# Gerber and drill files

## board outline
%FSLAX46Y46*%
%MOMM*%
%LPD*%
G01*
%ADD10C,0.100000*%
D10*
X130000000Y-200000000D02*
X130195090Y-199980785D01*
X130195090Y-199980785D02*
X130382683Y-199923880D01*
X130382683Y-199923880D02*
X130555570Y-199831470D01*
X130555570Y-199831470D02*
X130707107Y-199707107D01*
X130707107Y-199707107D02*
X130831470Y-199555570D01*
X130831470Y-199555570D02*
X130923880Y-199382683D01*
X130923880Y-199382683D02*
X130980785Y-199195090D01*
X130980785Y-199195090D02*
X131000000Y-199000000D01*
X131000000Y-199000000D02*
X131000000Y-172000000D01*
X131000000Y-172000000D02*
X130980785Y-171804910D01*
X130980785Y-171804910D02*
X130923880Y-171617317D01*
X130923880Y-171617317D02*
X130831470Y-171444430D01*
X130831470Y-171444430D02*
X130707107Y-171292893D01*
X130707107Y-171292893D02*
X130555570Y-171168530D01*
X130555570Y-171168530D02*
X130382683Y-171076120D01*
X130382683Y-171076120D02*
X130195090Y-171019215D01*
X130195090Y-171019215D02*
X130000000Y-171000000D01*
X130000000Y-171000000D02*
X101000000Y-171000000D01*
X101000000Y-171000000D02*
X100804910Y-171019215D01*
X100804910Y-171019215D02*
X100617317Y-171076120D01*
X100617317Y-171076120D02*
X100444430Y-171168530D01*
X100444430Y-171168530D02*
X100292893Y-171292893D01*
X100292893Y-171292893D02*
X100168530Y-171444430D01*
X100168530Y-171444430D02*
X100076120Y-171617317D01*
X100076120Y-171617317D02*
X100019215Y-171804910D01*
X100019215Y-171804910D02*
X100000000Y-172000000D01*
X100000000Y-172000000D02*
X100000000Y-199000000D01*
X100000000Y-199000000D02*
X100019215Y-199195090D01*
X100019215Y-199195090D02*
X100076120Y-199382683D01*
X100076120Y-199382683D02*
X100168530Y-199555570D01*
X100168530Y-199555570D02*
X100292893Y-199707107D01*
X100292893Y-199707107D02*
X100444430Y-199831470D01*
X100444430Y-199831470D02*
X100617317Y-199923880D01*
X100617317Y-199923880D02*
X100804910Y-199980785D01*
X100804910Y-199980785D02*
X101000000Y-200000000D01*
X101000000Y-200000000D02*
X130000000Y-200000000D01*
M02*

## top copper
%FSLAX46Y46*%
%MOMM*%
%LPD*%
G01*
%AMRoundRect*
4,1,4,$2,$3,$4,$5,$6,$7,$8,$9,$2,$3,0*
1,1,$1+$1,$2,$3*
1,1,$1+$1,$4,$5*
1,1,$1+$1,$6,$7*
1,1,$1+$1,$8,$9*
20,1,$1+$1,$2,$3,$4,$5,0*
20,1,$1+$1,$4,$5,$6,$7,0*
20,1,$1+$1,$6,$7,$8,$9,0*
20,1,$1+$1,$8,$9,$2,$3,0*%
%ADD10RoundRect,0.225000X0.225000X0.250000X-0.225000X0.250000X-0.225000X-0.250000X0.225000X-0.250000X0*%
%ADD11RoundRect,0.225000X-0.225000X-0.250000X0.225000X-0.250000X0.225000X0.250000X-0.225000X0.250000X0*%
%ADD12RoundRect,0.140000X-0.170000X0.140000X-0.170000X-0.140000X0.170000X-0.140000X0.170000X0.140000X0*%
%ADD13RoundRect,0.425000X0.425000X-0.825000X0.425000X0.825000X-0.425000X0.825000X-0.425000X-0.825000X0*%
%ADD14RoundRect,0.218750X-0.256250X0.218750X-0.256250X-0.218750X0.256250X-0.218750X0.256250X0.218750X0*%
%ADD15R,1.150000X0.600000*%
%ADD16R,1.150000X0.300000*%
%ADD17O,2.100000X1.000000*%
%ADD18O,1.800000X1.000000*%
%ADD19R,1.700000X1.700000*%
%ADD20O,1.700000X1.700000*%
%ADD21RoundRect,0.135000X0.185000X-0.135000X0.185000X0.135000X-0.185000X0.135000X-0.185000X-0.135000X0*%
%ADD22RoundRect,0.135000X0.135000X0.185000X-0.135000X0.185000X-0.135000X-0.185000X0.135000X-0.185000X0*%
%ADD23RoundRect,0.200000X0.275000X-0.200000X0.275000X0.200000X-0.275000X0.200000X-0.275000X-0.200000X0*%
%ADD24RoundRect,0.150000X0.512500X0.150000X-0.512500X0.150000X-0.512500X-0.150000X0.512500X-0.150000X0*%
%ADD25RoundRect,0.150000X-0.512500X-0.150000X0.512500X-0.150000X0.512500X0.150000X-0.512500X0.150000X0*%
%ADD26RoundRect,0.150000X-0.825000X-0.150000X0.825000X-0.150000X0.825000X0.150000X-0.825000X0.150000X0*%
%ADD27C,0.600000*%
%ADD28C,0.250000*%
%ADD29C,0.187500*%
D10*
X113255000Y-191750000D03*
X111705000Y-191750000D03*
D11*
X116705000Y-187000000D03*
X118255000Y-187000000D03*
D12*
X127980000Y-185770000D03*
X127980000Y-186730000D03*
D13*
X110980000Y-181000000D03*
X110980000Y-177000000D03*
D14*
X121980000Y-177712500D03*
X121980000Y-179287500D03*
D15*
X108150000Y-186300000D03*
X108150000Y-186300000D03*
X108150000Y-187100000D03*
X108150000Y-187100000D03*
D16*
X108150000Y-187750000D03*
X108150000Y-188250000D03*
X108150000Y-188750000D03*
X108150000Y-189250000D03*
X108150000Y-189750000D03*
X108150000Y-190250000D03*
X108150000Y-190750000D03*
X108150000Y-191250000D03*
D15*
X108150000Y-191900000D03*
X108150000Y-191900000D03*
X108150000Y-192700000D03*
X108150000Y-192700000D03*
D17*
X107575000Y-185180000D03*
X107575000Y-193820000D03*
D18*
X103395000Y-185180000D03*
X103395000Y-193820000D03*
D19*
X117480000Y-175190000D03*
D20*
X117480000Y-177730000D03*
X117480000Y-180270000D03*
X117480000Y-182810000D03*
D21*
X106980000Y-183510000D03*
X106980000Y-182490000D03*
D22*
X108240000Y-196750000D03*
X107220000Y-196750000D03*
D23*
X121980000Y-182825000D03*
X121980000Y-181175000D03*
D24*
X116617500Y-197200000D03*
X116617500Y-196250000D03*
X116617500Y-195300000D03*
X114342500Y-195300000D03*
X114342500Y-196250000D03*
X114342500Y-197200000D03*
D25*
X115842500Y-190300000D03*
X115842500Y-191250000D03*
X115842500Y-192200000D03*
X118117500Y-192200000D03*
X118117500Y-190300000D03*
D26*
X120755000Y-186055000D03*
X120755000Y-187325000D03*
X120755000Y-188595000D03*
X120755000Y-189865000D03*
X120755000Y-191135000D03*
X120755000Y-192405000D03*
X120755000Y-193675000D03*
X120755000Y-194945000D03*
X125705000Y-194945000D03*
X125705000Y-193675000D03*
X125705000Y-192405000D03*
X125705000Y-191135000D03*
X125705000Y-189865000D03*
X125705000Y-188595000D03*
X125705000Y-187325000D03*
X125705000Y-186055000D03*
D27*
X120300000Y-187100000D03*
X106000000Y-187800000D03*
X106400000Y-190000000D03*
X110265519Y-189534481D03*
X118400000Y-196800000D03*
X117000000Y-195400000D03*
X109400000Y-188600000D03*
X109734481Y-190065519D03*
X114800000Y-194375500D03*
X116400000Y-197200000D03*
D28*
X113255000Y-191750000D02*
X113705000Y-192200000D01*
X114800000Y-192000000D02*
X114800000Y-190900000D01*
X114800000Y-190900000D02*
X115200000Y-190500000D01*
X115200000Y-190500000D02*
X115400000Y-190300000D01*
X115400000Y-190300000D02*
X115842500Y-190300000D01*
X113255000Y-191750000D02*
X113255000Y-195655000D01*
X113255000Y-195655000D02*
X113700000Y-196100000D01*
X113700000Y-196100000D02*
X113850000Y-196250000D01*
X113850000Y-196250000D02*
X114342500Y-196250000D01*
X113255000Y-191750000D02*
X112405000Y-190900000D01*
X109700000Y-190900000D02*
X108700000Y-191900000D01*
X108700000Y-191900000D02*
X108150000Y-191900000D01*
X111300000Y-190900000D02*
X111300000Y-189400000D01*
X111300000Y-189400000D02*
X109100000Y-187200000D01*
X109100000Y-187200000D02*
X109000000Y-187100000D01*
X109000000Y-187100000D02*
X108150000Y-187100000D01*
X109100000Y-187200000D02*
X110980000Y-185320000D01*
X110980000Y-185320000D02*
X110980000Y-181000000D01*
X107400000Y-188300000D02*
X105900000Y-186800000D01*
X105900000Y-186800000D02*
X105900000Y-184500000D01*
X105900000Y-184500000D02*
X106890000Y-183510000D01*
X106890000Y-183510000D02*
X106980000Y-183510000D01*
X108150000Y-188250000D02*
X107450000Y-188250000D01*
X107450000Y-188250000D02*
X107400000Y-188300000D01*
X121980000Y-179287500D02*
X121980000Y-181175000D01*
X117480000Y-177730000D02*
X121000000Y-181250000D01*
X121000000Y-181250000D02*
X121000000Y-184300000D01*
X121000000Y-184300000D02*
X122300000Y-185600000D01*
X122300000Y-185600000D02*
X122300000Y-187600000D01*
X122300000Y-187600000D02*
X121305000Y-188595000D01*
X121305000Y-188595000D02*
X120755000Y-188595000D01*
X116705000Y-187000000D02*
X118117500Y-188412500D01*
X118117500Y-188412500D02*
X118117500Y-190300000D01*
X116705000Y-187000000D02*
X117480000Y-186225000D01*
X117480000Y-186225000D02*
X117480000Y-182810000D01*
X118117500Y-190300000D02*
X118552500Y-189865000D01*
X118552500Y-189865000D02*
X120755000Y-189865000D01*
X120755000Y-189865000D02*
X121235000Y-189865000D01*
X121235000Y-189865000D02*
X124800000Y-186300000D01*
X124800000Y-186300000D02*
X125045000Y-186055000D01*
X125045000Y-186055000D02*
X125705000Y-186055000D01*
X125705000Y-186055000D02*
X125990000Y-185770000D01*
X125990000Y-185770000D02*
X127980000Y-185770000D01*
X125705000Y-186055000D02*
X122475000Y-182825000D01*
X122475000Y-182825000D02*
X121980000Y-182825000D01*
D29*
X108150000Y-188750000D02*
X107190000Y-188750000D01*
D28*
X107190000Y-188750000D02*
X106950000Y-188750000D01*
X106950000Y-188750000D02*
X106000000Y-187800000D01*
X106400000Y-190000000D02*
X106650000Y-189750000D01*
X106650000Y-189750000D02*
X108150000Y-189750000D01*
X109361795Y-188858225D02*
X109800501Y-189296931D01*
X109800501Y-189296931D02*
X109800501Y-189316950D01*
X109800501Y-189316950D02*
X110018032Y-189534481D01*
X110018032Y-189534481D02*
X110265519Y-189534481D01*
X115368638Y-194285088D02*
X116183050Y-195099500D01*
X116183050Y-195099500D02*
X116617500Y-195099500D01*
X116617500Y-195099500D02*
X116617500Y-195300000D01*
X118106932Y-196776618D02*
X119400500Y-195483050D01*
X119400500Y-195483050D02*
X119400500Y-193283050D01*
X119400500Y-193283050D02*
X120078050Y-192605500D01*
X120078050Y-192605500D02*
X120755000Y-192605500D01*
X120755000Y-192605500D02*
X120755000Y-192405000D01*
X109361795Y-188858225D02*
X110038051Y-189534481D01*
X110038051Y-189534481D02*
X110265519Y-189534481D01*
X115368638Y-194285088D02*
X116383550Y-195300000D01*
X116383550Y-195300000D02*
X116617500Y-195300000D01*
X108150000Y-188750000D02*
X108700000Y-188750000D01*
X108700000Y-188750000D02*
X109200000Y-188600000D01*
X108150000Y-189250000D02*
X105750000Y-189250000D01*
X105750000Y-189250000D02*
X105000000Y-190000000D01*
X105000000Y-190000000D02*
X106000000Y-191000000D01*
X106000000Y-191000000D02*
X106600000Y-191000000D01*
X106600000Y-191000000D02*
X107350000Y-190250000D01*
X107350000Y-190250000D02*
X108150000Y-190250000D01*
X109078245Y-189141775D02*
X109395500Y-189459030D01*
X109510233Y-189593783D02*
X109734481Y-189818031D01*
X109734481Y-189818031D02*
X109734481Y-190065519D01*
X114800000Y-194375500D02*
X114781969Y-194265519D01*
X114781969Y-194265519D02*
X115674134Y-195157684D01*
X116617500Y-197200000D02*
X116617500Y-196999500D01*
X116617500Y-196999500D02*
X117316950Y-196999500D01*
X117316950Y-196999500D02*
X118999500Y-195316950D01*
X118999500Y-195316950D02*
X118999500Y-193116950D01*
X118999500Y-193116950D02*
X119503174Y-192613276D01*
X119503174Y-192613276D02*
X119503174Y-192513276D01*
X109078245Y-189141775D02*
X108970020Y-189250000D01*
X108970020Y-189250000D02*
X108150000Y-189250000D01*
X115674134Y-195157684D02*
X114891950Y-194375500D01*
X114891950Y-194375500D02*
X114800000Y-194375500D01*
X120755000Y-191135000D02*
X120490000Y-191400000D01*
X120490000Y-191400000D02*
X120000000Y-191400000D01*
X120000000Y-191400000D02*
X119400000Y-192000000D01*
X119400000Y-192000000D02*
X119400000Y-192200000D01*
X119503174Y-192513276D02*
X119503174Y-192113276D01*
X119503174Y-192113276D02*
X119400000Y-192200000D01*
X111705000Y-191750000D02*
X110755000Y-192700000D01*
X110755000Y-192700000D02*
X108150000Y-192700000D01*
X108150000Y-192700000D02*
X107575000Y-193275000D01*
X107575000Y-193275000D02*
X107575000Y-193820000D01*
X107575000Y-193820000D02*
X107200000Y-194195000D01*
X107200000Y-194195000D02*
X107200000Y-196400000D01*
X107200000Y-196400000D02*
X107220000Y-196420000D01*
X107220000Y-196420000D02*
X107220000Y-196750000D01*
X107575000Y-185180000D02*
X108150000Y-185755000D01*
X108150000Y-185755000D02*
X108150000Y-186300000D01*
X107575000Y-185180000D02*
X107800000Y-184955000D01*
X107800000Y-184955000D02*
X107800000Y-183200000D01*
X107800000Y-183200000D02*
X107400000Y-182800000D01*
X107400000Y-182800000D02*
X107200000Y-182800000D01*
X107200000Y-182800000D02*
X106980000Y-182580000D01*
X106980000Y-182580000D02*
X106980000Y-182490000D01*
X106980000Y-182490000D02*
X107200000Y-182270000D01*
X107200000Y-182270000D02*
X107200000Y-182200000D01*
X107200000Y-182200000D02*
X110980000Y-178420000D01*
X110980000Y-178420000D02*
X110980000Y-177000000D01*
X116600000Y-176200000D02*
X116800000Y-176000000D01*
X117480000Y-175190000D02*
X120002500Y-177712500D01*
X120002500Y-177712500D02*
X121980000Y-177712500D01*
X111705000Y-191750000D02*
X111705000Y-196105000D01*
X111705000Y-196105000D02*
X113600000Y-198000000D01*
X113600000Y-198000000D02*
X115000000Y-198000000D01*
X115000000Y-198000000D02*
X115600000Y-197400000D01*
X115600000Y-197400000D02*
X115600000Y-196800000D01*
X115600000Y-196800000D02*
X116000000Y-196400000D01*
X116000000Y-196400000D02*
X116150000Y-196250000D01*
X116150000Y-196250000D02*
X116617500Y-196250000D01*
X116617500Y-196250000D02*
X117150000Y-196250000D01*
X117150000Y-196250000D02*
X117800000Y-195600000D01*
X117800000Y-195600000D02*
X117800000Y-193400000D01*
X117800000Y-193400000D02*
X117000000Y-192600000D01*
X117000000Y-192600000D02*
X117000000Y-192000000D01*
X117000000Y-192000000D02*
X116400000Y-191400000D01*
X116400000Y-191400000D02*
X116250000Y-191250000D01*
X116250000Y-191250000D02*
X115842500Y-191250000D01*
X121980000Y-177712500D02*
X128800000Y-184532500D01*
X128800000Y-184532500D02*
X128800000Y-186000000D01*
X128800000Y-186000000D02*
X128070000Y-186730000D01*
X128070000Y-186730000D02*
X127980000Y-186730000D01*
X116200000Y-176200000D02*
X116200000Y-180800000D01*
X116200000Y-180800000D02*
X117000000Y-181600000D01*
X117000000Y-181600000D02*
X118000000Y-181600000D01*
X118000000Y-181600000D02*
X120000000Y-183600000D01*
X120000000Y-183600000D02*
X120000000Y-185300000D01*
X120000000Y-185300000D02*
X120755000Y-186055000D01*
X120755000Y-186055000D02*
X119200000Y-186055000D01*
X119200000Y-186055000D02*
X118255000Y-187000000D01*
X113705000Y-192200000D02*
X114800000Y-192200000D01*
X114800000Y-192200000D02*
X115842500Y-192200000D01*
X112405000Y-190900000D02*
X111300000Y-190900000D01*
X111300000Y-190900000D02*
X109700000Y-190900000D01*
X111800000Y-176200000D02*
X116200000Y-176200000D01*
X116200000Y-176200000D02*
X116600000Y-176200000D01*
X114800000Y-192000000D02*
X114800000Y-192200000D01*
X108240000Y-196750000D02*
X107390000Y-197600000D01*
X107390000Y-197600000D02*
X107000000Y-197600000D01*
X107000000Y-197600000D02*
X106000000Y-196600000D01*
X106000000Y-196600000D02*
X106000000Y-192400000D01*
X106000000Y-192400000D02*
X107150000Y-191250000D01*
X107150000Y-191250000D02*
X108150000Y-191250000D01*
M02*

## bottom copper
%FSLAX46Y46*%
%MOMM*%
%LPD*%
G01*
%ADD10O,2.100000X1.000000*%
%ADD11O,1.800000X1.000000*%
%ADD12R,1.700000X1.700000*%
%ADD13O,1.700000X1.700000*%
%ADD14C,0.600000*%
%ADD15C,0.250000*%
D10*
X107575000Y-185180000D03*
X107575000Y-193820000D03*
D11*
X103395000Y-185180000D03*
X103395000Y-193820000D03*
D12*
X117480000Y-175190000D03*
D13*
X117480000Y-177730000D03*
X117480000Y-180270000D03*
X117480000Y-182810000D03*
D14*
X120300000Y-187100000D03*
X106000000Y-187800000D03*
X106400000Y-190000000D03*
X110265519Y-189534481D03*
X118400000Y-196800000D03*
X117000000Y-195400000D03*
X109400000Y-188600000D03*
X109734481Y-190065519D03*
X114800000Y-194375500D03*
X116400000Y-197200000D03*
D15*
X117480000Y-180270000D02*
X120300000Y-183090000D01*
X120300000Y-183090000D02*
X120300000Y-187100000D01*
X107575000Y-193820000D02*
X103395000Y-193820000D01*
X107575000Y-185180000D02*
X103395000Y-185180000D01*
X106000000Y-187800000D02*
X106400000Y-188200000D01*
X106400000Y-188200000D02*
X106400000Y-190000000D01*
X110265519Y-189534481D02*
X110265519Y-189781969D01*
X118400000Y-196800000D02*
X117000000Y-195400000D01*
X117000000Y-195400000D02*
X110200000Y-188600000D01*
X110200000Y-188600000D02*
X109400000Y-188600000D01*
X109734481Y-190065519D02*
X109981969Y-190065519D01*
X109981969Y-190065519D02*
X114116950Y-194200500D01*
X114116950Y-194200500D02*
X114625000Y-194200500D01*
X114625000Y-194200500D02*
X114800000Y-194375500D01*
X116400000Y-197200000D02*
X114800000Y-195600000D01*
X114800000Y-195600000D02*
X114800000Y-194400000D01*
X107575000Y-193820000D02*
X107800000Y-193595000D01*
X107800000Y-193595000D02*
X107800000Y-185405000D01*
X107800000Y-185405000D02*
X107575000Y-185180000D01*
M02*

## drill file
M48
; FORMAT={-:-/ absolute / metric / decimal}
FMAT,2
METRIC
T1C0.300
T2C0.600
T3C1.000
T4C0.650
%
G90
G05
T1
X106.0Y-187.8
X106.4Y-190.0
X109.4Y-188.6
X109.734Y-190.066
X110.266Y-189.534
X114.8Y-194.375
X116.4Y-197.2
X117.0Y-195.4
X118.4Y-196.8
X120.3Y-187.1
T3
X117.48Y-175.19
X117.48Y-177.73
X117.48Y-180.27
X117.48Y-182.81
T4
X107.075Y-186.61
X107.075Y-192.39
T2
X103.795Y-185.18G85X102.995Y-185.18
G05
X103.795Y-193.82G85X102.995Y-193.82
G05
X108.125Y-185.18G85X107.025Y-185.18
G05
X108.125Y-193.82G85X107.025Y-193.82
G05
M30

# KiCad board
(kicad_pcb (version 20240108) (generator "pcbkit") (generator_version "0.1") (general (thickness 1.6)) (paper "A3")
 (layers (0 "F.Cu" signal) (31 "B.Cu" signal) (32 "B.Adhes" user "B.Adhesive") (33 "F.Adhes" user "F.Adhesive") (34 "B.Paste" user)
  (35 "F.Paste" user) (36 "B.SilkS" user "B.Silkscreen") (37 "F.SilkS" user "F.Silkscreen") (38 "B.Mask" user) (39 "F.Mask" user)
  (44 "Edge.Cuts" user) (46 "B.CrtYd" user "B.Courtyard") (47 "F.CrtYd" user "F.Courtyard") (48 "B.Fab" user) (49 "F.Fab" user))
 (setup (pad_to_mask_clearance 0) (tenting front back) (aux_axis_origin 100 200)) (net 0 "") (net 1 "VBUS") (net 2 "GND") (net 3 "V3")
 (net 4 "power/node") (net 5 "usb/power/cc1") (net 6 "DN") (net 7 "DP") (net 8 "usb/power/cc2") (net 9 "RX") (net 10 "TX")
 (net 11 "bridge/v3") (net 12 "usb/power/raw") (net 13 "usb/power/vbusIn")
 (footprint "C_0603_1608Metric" (layer "F.Cu") (at 112.48 191.75 180)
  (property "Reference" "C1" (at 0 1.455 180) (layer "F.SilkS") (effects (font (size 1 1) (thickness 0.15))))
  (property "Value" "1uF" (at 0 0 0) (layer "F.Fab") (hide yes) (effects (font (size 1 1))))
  (pad "1" smd roundrect (at -0.775 0 180) (size 0.9 0.95) (layers "F.Cu" "F.Paste" "F.Mask") (roundrect_rratio 0.250000000000)
   (solder_mask_margin 0.05) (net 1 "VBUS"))
  (pad "2" smd roundrect (at 0.775 0 180) (size 0.9 0.95) (layers "F.Cu" "F.Paste" "F.Mask") (roundrect_rratio 0.250000000000)
   (solder_mask_margin 0.05) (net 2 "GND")))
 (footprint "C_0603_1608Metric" (layer "F.Cu") (at 117.48 187 0)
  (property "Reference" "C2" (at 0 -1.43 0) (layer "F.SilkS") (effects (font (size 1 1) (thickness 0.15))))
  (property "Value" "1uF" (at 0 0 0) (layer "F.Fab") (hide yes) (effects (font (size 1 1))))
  (pad "1" smd roundrect (at -0.775 0 0) (size 0.9 0.95) (layers "F.Cu" "F.Paste" "F.Mask") (roundrect_rratio 0.250000000000)
   (solder_mask_margin 0.05) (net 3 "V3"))
  (pad "2" smd roundrect (at 0.775 0 0) (size 0.9 0.95) (layers "F.Cu" "F.Paste" "F.Mask") (roundrect_rratio 0.250000000000)
   (solder_mask_margin 0.05) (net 2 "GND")))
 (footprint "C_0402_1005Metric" (layer "F.Cu") (at 127.98 186.25 270)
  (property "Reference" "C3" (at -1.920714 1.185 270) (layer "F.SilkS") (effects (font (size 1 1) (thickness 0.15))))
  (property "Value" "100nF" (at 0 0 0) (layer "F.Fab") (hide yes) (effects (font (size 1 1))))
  (pad "1" smd roundrect (at -0.48 0 270) (size 0.56 0.62) (layers "F.Cu" "F.Paste" "F.Mask") (roundrect_rratio 0.250000000000)
   (solder_mask_margin 0.05) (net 3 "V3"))
  (pad "2" smd roundrect (at 0.48 0 270) (size 0.56 0.62) (layers "F.Cu" "F.Paste" "F.Mask") (roundrect_rratio 0.250000000000)
   (solder_mask_margin 0.05) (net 2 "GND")))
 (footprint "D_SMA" (layer "F.Cu") (at 110.98 179 90)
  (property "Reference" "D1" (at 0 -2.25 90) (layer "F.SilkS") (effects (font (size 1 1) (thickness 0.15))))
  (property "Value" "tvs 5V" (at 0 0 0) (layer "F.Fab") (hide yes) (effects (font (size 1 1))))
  (pad "1" smd roundrect (at -2 0 90) (size 2.5 1.7) (layers "F.Cu" "F.Paste" "F.Mask") (roundrect_rratio 0.250000000000)
   (solder_mask_margin 0.05) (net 1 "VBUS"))
  (pad "2" smd roundrect (at 2 0 90) (size 2.5 1.7) (layers "F.Cu" "F.Paste" "F.Mask") (roundrect_rratio 0.250000000000)
   (solder_mask_margin 0.05) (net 2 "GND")))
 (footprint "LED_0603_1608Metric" (layer "F.Cu") (at 121.98 178.5 270)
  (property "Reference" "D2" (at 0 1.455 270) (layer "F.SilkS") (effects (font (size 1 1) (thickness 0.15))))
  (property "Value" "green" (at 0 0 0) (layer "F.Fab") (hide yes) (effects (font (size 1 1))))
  (pad "1" smd roundrect (at -0.7875 0 270) (size 0.875 0.95) (layers "F.Cu" "F.Paste" "F.Mask") (roundrect_rratio 0.250000000000)
   (solder_mask_margin 0.05) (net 2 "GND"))
  (pad "2" smd roundrect (at 0.7875 0 270) (size 0.875 0.95) (layers "F.Cu" "F.Paste" "F.Mask") (roundrect_rratio 0.250000000000)
   (solder_mask_margin 0.05) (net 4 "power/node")))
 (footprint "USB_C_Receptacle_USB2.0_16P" (layer "F.Cu") (at 108.15 189.5 270)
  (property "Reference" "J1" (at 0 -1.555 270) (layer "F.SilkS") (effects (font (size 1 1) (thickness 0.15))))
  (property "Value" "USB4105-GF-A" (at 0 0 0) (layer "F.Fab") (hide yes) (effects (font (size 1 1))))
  (pad "A1" smd rect (at -3.2 0 270) (size 0.6 1.15) (layers "F.Cu" "F.Paste" "F.Mask") (solder_mask_margin 0.05) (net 2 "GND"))
  (pad "B12" smd rect (at -3.2 0 270) (size 0.6 1.15) (layers "F.Cu" "F.Paste" "F.Mask") (solder_mask_margin 0.05) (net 2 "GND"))
  (pad "A4" smd rect (at -2.4 0 270) (size 0.6 1.15) (layers "F.Cu" "F.Paste" "F.Mask") (solder_mask_margin 0.05) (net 1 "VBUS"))
  (pad "B9" smd rect (at -2.4 0 270) (size 0.6 1.15) (layers "F.Cu" "F.Paste" "F.Mask") (solder_mask_margin 0.05) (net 1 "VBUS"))
  (pad "B8" smd rect (at -1.75 0 270) (size 0.3 1.15) (layers "F.Cu" "F.Paste" "F.Mask") (solder_mask_margin 0.05))
  (pad "A5" smd rect (at -1.25 0 270) (size 0.3 1.15) (layers "F.Cu" "F.Paste" "F.Mask") (solder_mask_margin 0.05) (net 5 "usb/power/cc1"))
  (pad "B7" smd rect (at -0.75 0 270) (size 0.3 1.15) (layers "F.Cu" "F.Paste" "F.Mask") (solder_mask_margin 0.05) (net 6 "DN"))
  (pad "A6" smd rect (at -0.25 0 270) (size 0.3 1.15) (layers "F.Cu" "F.Paste" "F.Mask") (solder_mask_margin 0.05) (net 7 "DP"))
  (pad "A7" smd rect (at 0.25 0 270) (size 0.3 1.15) (layers "F.Cu" "F.Paste" "F.Mask") (solder_mask_margin 0.05) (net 6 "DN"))
  (pad "B6" smd rect (at 0.75 0 270) (size 0.3 1.15) (layers "F.Cu" "F.Paste" "F.Mask") (solder_mask_margin 0.05) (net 7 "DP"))
  (pad "A8" smd rect (at 1.25 0 270) (size 0.3 1.15) (layers "F.Cu" "F.Paste" "F.Mask") (solder_mask_margin 0.05))
  (pad "B5" smd rect (at 1.75 0 270) (size 0.3 1.15) (layers "F.Cu" "F.Paste" "F.Mask") (solder_mask_margin 0.05) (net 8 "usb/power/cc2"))
  (pad "B4" smd rect (at 2.4 0 270) (size 0.6 1.15) (layers "F.Cu" "F.Paste" "F.Mask") (solder_mask_margin 0.05) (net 1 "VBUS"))
  (pad "A9" smd rect (at 2.4 0 270) (size 0.6 1.15) (layers "F.Cu" "F.Paste" "F.Mask") (solder_mask_margin 0.05) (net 1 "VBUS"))
  (pad "B1" smd rect (at 3.2 0 270) (size 0.6 1.15) (layers "F.Cu" "F.Paste" "F.Mask") (solder_mask_margin 0.05) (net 2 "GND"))
  (pad "A12" smd rect (at 3.2 0 270) (size 0.6 1.15) (layers "F.Cu" "F.Paste" "F.Mask") (solder_mask_margin 0.05) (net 2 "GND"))
  (pad "S1" thru_hole oval (at -4.32 0.575 270) (size 1 2.1) (drill oval 0.6 1.7) (layers "*.Cu" "*.Mask") (solder_mask_margin 0.05)
   (zone_connect 2) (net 2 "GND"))
  (pad "S1" thru_hole oval (at 4.32 0.575 270) (size 1 2.1) (drill oval 0.6 1.7) (layers "*.Cu" "*.Mask") (solder_mask_margin 0.05)
   (zone_connect 2) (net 2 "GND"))
  (pad "S1" thru_hole oval (at -4.32 4.755 270) (size 1 1.8) (drill oval 0.6 1.4) (layers "*.Cu" "*.Mask") (solder_mask_margin 0.05)
   (zone_connect 2) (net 2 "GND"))
  (pad "S1" thru_hole oval (at 4.32 4.755 270) (size 1 1.8) (drill oval 0.6 1.4) (layers "*.Cu" "*.Mask") (solder_mask_margin 0.05)
   (zone_connect 2) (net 2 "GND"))
  (pad "" np_thru_hole circle (at -2.89 1.075 270) (size 0.65 0.65) (drill 0.65) (layers "*.Cu" "*.Mask") (solder_mask_margin 0.05))
  (pad "" np_thru_hole circle (at 2.89 1.075 270) (size 0.65 0.65) (drill 0.65) (layers "*.Cu" "*.Mask") (solder_mask_margin 0.05)))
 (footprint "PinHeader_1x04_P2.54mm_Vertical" (layer "F.Cu") (at 117.48 179 0)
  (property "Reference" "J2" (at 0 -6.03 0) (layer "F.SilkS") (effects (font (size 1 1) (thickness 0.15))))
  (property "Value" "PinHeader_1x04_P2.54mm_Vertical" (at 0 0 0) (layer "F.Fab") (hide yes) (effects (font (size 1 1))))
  (pad "1" thru_hole rect (at 0 -3.81 0) (size 1.7 1.7) (drill 1) (layers "*.Cu" "*.Mask") (solder_mask_margin 0.05) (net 2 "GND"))
  (pad "2" thru_hole oval (at 0 -1.27 0) (size 1.7 1.7) (drill 1) (layers "*.Cu" "*.Mask") (solder_mask_margin 0.05) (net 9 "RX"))
  (pad "3" thru_hole oval (at 0 1.27 0) (size 1.7 1.7) (drill 1) (layers "*.Cu" "*.Mask") (solder_mask_margin 0.05) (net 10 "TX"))
  (pad "4" thru_hole oval (at 0 3.81 0) (size 1.7 1.7) (drill 1) (layers "*.Cu" "*.Mask") (solder_mask_margin 0.05) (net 3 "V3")))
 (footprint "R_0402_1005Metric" (layer "F.Cu") (at 106.98 183 90)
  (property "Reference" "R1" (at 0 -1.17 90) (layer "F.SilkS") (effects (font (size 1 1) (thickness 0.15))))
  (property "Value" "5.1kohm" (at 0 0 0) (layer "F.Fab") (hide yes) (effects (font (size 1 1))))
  (pad "1" smd roundrect (at -0.51 0 90) (size 0.54 0.64) (layers "F.Cu" "F.Paste" "F.Mask") (roundrect_rratio 0.250000000000)
   (solder_mask_margin 0.05) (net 5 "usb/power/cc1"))
  (pad "2" smd roundrect (at 0.51 0 90) (size 0.54 0.64) (layers "F.Cu" "F.Paste" "F.Mask") (roundrect_rratio 0.250000000000)
   (solder_mask_margin 0.05) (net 2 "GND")))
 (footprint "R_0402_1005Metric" (layer "F.Cu") (at 107.73 196.75 180)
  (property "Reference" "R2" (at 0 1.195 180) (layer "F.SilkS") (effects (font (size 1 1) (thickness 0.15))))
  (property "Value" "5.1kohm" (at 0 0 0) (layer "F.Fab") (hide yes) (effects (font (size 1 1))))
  (pad "1" smd roundrect (at -0.51 0 180) (size 0.54 0.64) (layers "F.Cu" "F.Paste" "F.Mask") (roundrect_rratio 0.250000000000)
   (solder_mask_margin 0.05) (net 8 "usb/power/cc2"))
  (pad "2" smd roundrect (at 0.51 0 180) (size 0.54 0.64) (layers "F.Cu" "F.Paste" "F.Mask") (roundrect_rratio 0.250000000000)
   (solder_mask_margin 0.05) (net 2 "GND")))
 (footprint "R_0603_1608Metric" (layer "F.Cu") (at 121.98 182 90)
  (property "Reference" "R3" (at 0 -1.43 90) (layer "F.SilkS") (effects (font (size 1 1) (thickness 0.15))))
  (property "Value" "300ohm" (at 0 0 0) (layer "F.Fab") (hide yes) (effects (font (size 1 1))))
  (pad "1" smd roundrect (at -0.825 0 90) (size 0.8 0.95) (layers "F.Cu" "F.Paste" "F.Mask") (roundrect_rratio 0.250000000000)
   (solder_mask_margin 0.05) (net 3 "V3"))
  (pad "2" smd roundrect (at 0.825 0 90) (size 0.8 0.95) (layers "F.Cu" "F.Paste" "F.Mask") (roundrect_rratio 0.250000000000)
   (solder_mask_margin 0.05) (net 4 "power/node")))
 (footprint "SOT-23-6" (layer "F.Cu") (at 115.48 196.25 180)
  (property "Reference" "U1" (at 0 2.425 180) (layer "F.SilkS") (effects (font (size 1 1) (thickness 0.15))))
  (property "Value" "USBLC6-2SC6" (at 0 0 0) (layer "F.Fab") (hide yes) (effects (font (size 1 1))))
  (pad "1" smd roundrect (at -1.1375 -0.95 180) (size 1.325 0.6) (layers "F.Cu" "F.Paste" "F.Mask") (roundrect_rratio 0.250000000000)
   (solder_mask_margin 0.05) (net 7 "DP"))
  (pad "2" smd roundrect (at -1.1375 0 180) (size 1.325 0.6) (layers "F.Cu" "F.Paste" "F.Mask") (roundrect_rratio 0.250000000000)
   (solder_mask_margin 0.05) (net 2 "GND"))
  (pad "3" smd roundrect (at -1.1375 0.95 180) (size 1.325 0.6) (layers "F.Cu" "F.Paste" "F.Mask") (roundrect_rratio 0.250000000000)
   (solder_mask_margin 0.05) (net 6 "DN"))
  (pad "4" smd roundrect (at 1.1375 0.95 180) (size 1.325 0.6) (layers "F.Cu" "F.Paste" "F.Mask") (roundrect_rratio 0.250000000000)
   (solder_mask_margin 0.05))
  (pad "5" smd roundrect (at 1.1375 0 180) (size 1.325 0.6) (layers "F.Cu" "F.Paste" "F.Mask") (roundrect_rratio 0.250000000000)
   (solder_mask_margin 0.05) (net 1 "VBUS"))
  (pad "6" smd roundrect (at 1.1375 -0.95 180) (size 1.325 0.6) (layers "F.Cu" "F.Paste" "F.Mask") (roundrect_rratio 0.250000000000)
   (solder_mask_margin 0.05)))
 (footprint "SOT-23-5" (layer "F.Cu") (at 116.98 191.25 0)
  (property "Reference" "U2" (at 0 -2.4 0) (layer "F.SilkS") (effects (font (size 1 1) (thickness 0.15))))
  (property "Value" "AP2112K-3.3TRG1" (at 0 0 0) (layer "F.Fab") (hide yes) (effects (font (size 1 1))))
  (pad "1" smd roundrect (at -1.1375 -0.95 0) (size 1.325 0.6) (layers "F.Cu" "F.Paste" "F.Mask") (roundrect_rratio 0.250000000000)
   (solder_mask_margin 0.05) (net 1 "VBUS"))
  (pad "2" smd roundrect (at -1.1375 0 0) (size 1.325 0.6) (layers "F.Cu" "F.Paste" "F.Mask") (roundrect_rratio 0.250000000000)
   (solder_mask_margin 0.05) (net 2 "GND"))
  (pad "3" smd roundrect (at -1.1375 0.95 0) (size 1.325 0.6) (layers "F.Cu" "F.Paste" "F.Mask") (roundrect_rratio 0.250000000000)
   (solder_mask_margin 0.05) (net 1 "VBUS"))
  (pad "4" smd roundrect (at 1.1375 0.95 0) (size 1.325 0.6) (layers "F.Cu" "F.Paste" "F.Mask") (roundrect_rratio 0.250000000000)
   (solder_mask_margin 0.05))
  (pad "5" smd roundrect (at 1.1375 -0.95 0) (size 1.325 0.6) (layers "F.Cu" "F.Paste" "F.Mask") (roundrect_rratio 0.250000000000)
   (solder_mask_margin 0.05) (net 3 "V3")))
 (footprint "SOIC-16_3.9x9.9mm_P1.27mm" (layer "F.Cu") (at 123.23 190.5 0)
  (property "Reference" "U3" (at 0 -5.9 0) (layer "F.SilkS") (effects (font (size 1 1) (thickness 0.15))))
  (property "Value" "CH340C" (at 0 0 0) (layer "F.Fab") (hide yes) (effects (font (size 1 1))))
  (pad "1" smd roundrect (at -2.475 -4.445 0) (size 1.95 0.6) (layers "F.Cu" "F.Paste" "F.Mask") (roundrect_rratio 0.250000000000)
   (solder_mask_margin 0.05) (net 2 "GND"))
  (pad "2" smd roundrect (at -2.475 -3.175 0) (size 1.95 0.6) (layers "F.Cu" "F.Paste" "F.Mask") (roundrect_rratio 0.250000000000)
   (solder_mask_margin 0.05) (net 10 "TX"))
  (pad "3" smd roundrect (at -2.475 -1.905 0) (size 1.95 0.6) (layers "F.Cu" "F.Paste" "F.Mask") (roundrect_rratio 0.250000000000)
   (solder_mask_margin 0.05) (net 9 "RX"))
  (pad "4" smd roundrect (at -2.475 -0.635 0) (size 1.95 0.6) (layers "F.Cu" "F.Paste" "F.Mask") (roundrect_rratio 0.250000000000)
   (solder_mask_margin 0.05) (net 3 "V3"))
  (pad "5" smd roundrect (at -2.475 0.635 0) (size 1.95 0.6) (layers "F.Cu" "F.Paste" "F.Mask") (roundrect_rratio 0.250000000000)
   (solder_mask_margin 0.05) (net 7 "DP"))
  (pad "6" smd roundrect (at -2.475 1.905 0) (size 1.95 0.6) (layers "F.Cu" "F.Paste" "F.Mask") (roundrect_rratio 0.250000000000)
   (solder_mask_margin 0.05) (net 6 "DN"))
  (pad "7" smd roundrect (at -2.475 3.175 0) (size 1.95 0.6) (layers "F.Cu" "F.Paste" "F.Mask") (roundrect_rratio 0.250000000000)
   (solder_mask_margin 0.05))
  (pad "8" smd roundrect (at -2.475 4.445 0) (size 1.95 0.6) (layers "F.Cu" "F.Paste" "F.Mask") (roundrect_rratio 0.250000000000)
   (solder_mask_margin 0.05))
  (pad "9" smd roundrect (at 2.475 4.445 0) (size 1.95 0.6) (layers "F.Cu" "F.Paste" "F.Mask") (roundrect_rratio 0.250000000000)
   (solder_mask_margin 0.05))
  (pad "10" smd roundrect (at 2.475 3.175 0) (size 1.95 0.6) (layers "F.Cu" "F.Paste" "F.Mask") (roundrect_rratio 0.250000000000)
   (solder_mask_margin 0.05))
  (pad "11" smd roundrect (at 2.475 1.905 0) (size 1.95 0.6) (layers "F.Cu" "F.Paste" "F.Mask") (roundrect_rratio 0.250000000000)
   (solder_mask_margin 0.05))
  (pad "12" smd roundrect (at 2.475 0.635 0) (size 1.95 0.6) (layers "F.Cu" "F.Paste" "F.Mask") (roundrect_rratio 0.250000000000)
   (solder_mask_margin 0.05))
  (pad "13" smd roundrect (at 2.475 -0.635 0) (size 1.95 0.6) (layers "F.Cu" "F.Paste" "F.Mask") (roundrect_rratio 0.250000000000)
   (solder_mask_margin 0.05))
  (pad "14" smd roundrect (at 2.475 -1.905 0) (size 1.95 0.6) (layers "F.Cu" "F.Paste" "F.Mask") (roundrect_rratio 0.250000000000)
   (solder_mask_margin 0.05))
  (pad "15" smd roundrect (at 2.475 -3.175 0) (size 1.95 0.6) (layers "F.Cu" "F.Paste" "F.Mask") (roundrect_rratio 0.250000000000)
   (solder_mask_margin 0.05))
  (pad "16" smd roundrect (at 2.475 -4.445 0) (size 1.95 0.6) (layers "F.Cu" "F.Paste" "F.Mask") (roundrect_rratio 0.250000000000)
   (solder_mask_margin 0.05) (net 3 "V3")))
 (gr_line (start 130 200) (end 130.19509 199.980785) (stroke (width 0.1) (type solid)) (layer "Edge.Cuts"))
 (gr_line (start 130.19509 199.980785) (end 130.382683 199.92388) (stroke (width 0.1) (type solid)) (layer "Edge.Cuts"))
 (gr_line (start 130.382683 199.92388) (end 130.55557 199.83147) (stroke (width 0.1) (type solid)) (layer "Edge.Cuts"))
 (gr_line (start 130.55557 199.83147) (end 130.707107 199.707107) (stroke (width 0.1) (type solid)) (layer "Edge.Cuts"))
 (gr_line (start 130.707107 199.707107) (end 130.83147 199.55557) (stroke (width 0.1) (type solid)) (layer "Edge.Cuts"))
 (gr_line (start 130.83147 199.55557) (end 130.92388 199.382683) (stroke (width 0.1) (type solid)) (layer "Edge.Cuts"))
 (gr_line (start 130.92388 199.382683) (end 130.980785 199.19509) (stroke (width 0.1) (type solid)) (layer "Edge.Cuts"))
 (gr_line (start 130.980785 199.19509) (end 131 199) (stroke (width 0.1) (type solid)) (layer "Edge.Cuts"))
 (gr_line (start 131 199) (end 131 172) (stroke (width 0.1) (type solid)) (layer "Edge.Cuts"))
 (gr_line (start 131 172) (end 130.980785 171.80491) (stroke (width 0.1) (type solid)) (layer "Edge.Cuts"))
 (gr_line (start 130.980785 171.80491) (end 130.92388 171.617317) (stroke (width 0.1) (type solid)) (layer "Edge.Cuts"))
 (gr_line (start 130.92388 171.617317) (end 130.83147 171.44443) (stroke (width 0.1) (type solid)) (layer "Edge.Cuts"))
 (gr_line (start 130.83147 171.44443) (end 130.707107 171.292893) (stroke (width 0.1) (type solid)) (layer "Edge.Cuts"))
 (gr_line (start 130.707107 171.292893) (end 130.55557 171.16853) (stroke (width 0.1) (type solid)) (layer "Edge.Cuts"))
 (gr_line (start 130.55557 171.16853) (end 130.382683 171.07612) (stroke (width 0.1) (type solid)) (layer "Edge.Cuts"))
 (gr_line (start 130.382683 171.07612) (end 130.19509 171.019215) (stroke (width 0.1) (type solid)) (layer "Edge.Cuts"))
 (gr_line (start 130.19509 171.019215) (end 130 171) (stroke (width 0.1) (type solid)) (layer "Edge.Cuts"))
 (gr_line (start 130 171) (end 101 171) (stroke (width 0.1) (type solid)) (layer "Edge.Cuts"))
 (gr_line (start 101 171) (end 100.80491 171.019215) (stroke (width 0.1) (type solid)) (layer "Edge.Cuts"))
 (gr_line (start 100.80491 171.019215) (end 100.617317 171.07612) (stroke (width 0.1) (type solid)) (layer "Edge.Cuts"))
 (gr_line (start 100.617317 171.07612) (end 100.44443 171.16853) (stroke (width 0.1) (type solid)) (layer "Edge.Cuts"))
 (gr_line (start 100.44443 171.16853) (end 100.292893 171.292893) (stroke (width 0.1) (type solid)) (layer "Edge.Cuts"))
 (gr_line (start 100.292893 171.292893) (end 100.16853 171.44443) (stroke (width 0.1) (type solid)) (layer "Edge.Cuts"))
 (gr_line (start 100.16853 171.44443) (end 100.07612 171.617317) (stroke (width 0.1) (type solid)) (layer "Edge.Cuts"))
 (gr_line (start 100.07612 171.617317) (end 100.019215 171.80491) (stroke (width 0.1) (type solid)) (layer "Edge.Cuts"))
 (gr_line (start 100.019215 171.80491) (end 100 172) (stroke (width 0.1) (type solid)) (layer "Edge.Cuts"))
 (gr_line (start 100 172) (end 100 199) (stroke (width 0.1) (type solid)) (layer "Edge.Cuts"))
 (gr_line (start 100 199) (end 100.019215 199.19509) (stroke (width 0.1) (type solid)) (layer "Edge.Cuts"))
 (gr_line (start 100.019215 199.19509) (end 100.07612 199.382683) (stroke (width 0.1) (type solid)) (layer "Edge.Cuts"))
 (gr_line (start 100.07612 199.382683) (end 100.16853 199.55557) (stroke (width 0.1) (type solid)) (layer "Edge.Cuts"))
 (gr_line (start 100.16853 199.55557) (end 100.292893 199.707107) (stroke (width 0.1) (type solid)) (layer "Edge.Cuts"))
 (gr_line (start 100.292893 199.707107) (end 100.44443 199.83147) (stroke (width 0.1) (type solid)) (layer "Edge.Cuts"))
 (gr_line (start 100.44443 199.83147) (end 100.617317 199.92388) (stroke (width 0.1) (type solid)) (layer "Edge.Cuts"))
 (gr_line (start 100.617317 199.92388) (end 100.80491 199.980785) (stroke (width 0.1) (type solid)) (layer "Edge.Cuts"))
 (gr_line (start 100.80491 199.980785) (end 101 200) (stroke (width 0.1) (type solid)) (layer "Edge.Cuts"))
 (gr_line (start 101 200) (end 130 200) (stroke (width 0.1) (type solid)) (layer "Edge.Cuts"))
 (segment (start 113.255 191.75) (end 113.705 192.2) (width 0.25) (layer "F.Cu") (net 1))
 (segment (start 114.8 192) (end 114.8 190.9) (width 0.25) (layer "F.Cu") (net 1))
 (segment (start 114.8 190.9) (end 115.2 190.5) (width 0.25) (layer "F.Cu") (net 1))
 (segment (start 115.2 190.5) (end 115.4 190.3) (width 0.25) (layer "F.Cu") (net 1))
 (segment (start 115.4 190.3) (end 115.8425 190.3) (width 0.25) (layer "F.Cu") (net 1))
 (segment (start 113.255 191.75) (end 113.255 195.655) (width 0.25) (layer "F.Cu") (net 1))
 (segment (start 113.255 195.655) (end 113.7 196.1) (width 0.25) (layer "F.Cu") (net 1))
 (segment (start 113.7 196.1) (end 113.85 196.25) (width 0.25) (layer "F.Cu") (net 1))
 (segment (start 113.85 196.25) (end 114.3425 196.25) (width 0.25) (layer "F.Cu") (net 1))
 (segment (start 113.255 191.75) (end 112.405 190.9) (width 0.25) (layer "F.Cu") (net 1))
 (segment (start 109.7 190.9) (end 108.7 191.9) (width 0.25) (layer "F.Cu") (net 1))
 (segment (start 108.7 191.9) (end 108.15 191.9) (width 0.25) (layer "F.Cu") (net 1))
 (segment (start 111.3 190.9) (end 111.3 189.4) (width 0.25) (layer "F.Cu") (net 1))
 (segment (start 111.3 189.4) (end 109.1 187.2) (width 0.25) (layer "F.Cu") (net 1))
 (segment (start 109.1 187.2) (end 109 187.1) (width 0.25) (layer "F.Cu") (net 1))
 (segment (start 109 187.1) (end 108.15 187.1) (width 0.25) (layer "F.Cu") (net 1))
 (segment (start 109.1 187.2) (end 110.98 185.32) (width 0.25) (layer "F.Cu") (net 1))
 (segment (start 110.98 185.32) (end 110.98 181) (width 0.25) (layer "F.Cu") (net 1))
 (segment (start 107.4 188.3) (end 105.9 186.8) (width 0.25) (layer "F.Cu") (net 5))
 (segment (start 105.9 186.8) (end 105.9 184.5) (width 0.25) (layer "F.Cu") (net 5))
 (segment (start 105.9 184.5) (end 106.89 183.51) (width 0.25) (layer "F.Cu") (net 5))
 (segment (start 106.89 183.51) (end 106.98 183.51) (width 0.25) (layer "F.Cu") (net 5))
 (segment (start 108.15 188.25) (end 107.45 188.25) (width 0.25) (layer "F.Cu") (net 5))
 (segment (start 107.45 188.25) (end 107.4 188.3) (width 0.25) (layer "F.Cu") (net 5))
 (segment (start 121.98 179.2875) (end 121.98 181.175) (width 0.25) (layer "F.Cu") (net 4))
 (segment (start 117.48 177.73) (end 121 181.25) (width 0.25) (layer "F.Cu") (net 9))
 (segment (start 121 181.25) (end 121 184.3) (width 0.25) (layer "F.Cu") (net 9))
 (segment (start 121 184.3) (end 122.3 185.6) (width 0.25) (layer "F.Cu") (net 9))
 (segment (start 122.3 185.6) (end 122.3 187.6) (width 0.25) (layer "F.Cu") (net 9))
 (segment (start 122.3 187.6) (end 121.305 188.595) (width 0.25) (layer "F.Cu") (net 9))
 (segment (start 121.305 188.595) (end 120.755 188.595) (width 0.25) (layer "F.Cu") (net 9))
 (segment (start 117.48 180.27) (end 120.3 183.09) (width 0.25) (layer "B.Cu") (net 10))
 (segment (start 120.3 183.09) (end 120.3 187.1) (width 0.25) (layer "B.Cu") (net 10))
 (segment (start 116.705 187) (end 118.1175 188.4125) (width 0.25) (layer "F.Cu") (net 3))
 (segment (start 118.1175 188.4125) (end 118.1175 190.3) (width 0.25) (layer "F.Cu") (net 3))
 (segment (start 116.705 187) (end 117.48 186.225) (width 0.25) (layer "F.Cu") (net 3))
 (segment (start 117.48 186.225) (end 117.48 182.81) (width 0.25) (layer "F.Cu") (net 3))
 (segment (start 118.1175 190.3) (end 118.5525 189.865) (width 0.25) (layer "F.Cu") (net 3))
 (segment (start 118.5525 189.865) (end 120.755 189.865) (width 0.25) (layer "F.Cu") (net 3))
 (segment (start 120.755 189.865) (end 121.235 189.865) (width 0.25) (layer "F.Cu") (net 3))
 (segment (start 121.235 189.865) (end 124.8 186.3) (width 0.25) (layer "F.Cu") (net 3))
 (segment (start 124.8 186.3) (end 125.045 186.055) (width 0.25) (layer "F.Cu") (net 3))
 (segment (start 125.045 186.055) (end 125.705 186.055) (width 0.25) (layer "F.Cu") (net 3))
 (segment (start 125.705 186.055) (end 125.99 185.77) (width 0.25) (layer "F.Cu") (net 3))
 (segment (start 125.99 185.77) (end 127.98 185.77) (width 0.25) (layer "F.Cu") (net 3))
 (segment (start 125.705 186.055) (end 122.475 182.825) (width 0.25) (layer "F.Cu") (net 3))
 (segment (start 122.475 182.825) (end 121.98 182.825) (width 0.25) (layer "F.Cu") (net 3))
 (via (at 120.3 187.1) (size 0.6) (drill 0.3) (layers "F.Cu" "B.Cu") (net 10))
 (segment (start 107.575 193.82) (end 103.395 193.82) (width 0.25) (layer "B.Cu") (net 2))
 (segment (start 107.575 185.18) (end 103.395 185.18) (width 0.25) (layer "B.Cu") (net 2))
 (segment (start 108.15 188.75) (end 107.19 188.75) (width 0.1875) (layer "F.Cu") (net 6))
 (segment (start 107.19 188.75) (end 106.95 188.75) (width 0.25) (layer "F.Cu") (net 6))
 (segment (start 106.95 188.75) (end 106 187.8) (width 0.25) (layer "F.Cu") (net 6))
 (segment (start 106 187.8) (end 106.4 188.2) (width 0.25) (layer "B.Cu") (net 6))
 (segment (start 106.4 188.2) (end 106.4 190) (width 0.25) (layer "B.Cu") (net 6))
 (segment (start 106.4 190) (end 106.65 189.75) (width 0.25) (layer "F.Cu") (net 6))
 (segment (start 106.65 189.75) (end 108.15 189.75) (width 0.25) (layer "F.Cu") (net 6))
 (segment (start 109.361795 188.858225) (end 109.800501 189.296931) (width 0.25) (layer "F.Cu") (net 6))
 (segment (start 109.800501 189.296931) (end 109.800501 189.31695) (width 0.25) (layer "F.Cu") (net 6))
 (segment (start 109.800501 189.31695) (end 110.018032 189.534481) (width 0.25) (layer "F.Cu") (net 6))
 (segment (start 110.018032 189.534481) (end 110.265519 189.534481) (width 0.25) (layer "F.Cu") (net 6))
 (segment (start 110.265519 189.534481) (end 110.265519 189.781969) (width 0.25) (layer "B.Cu") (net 6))
 (segment (start 115.368638 194.285088) (end 116.18305 195.0995) (width 0.25) (layer "F.Cu") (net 6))
 (segment (start 116.18305 195.0995) (end 116.6175 195.0995) (width 0.25) (layer "F.Cu") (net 6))
 (segment (start 116.6175 195.0995) (end 116.6175 195.3) (width 0.25) (layer "F.Cu") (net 6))
 (segment (start 118.106932 196.776618) (end 119.4005 195.48305) (width 0.25) (layer "F.Cu") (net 6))
 (segment (start 119.4005 195.48305) (end 119.4005 193.28305) (width 0.25) (layer "F.Cu") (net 6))
 (segment (start 119.4005 193.28305) (end 120.07805 192.6055) (width 0.25) (layer "F.Cu") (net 6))
 (segment (start 120.07805 192.6055) (end 120.755 192.6055) (width 0.25) (layer "F.Cu") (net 6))
 (segment (start 120.755 192.6055) (end 120.755 192.405) (width 0.25) (layer "F.Cu") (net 6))
 (segment (start 109.361795 188.858225) (end 110.038051 189.534481) (width 0.25) (layer "F.Cu") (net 6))
 (segment (start 110.038051 189.534481) (end 110.265519 189.534481) (width 0.25) (layer "F.Cu") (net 6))
 (segment (start 115.368638 194.285088) (end 116.38355 195.3) (width 0.25) (layer "F.Cu") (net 6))
 (segment (start 116.38355 195.3) (end 116.6175 195.3) (width 0.25) (layer "F.Cu") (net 6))
 (segment (start 118.4 196.8) (end 117 195.4) (width 0.25) (layer "B.Cu") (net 6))
 (segment (start 117 195.4) (end 110.2 188.6) (width 0.25) (layer "B.Cu") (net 6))
 (segment (start 110.2 188.6) (end 109.4 188.6) (width 0.25) (layer "B.Cu") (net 6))
 (segment (start 108.15 188.75) (end 108.7 188.75) (width 0.25) (layer "F.Cu") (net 6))
 (segment (start 108.7 188.75) (end 109.2 188.6) (width 0.25) (layer "F.Cu") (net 6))
 (segment (start 108.15 189.25) (end 105.75 189.25) (width 0.25) (layer "F.Cu") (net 7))
 (segment (start 105.75 189.25) (end 105 190) (width 0.25) (layer "F.Cu") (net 7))
 (segment (start 105 190) (end 106 191) (width 0.25) (layer "F.Cu") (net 7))
 (segment (start 106 191) (end 106.6 191) (width 0.25) (layer "F.Cu") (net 7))
 (segment (start 106.6 191) (end 107.35 190.25) (width 0.25) (layer "F.Cu") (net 7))
 (segment (start 107.35 190.25) (end 108.15 190.25) (width 0.25) (layer "F.Cu") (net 7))
 (segment (start 109.078245 189.141775) (end 109.3955 189.45903) (width 0.25) (layer "F.Cu") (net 7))
 (segment (start 109.510233 189.593783) (end 109.734481 189.818031) (width 0.25) (layer "F.Cu") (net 7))
 (segment (start 109.734481 189.818031) (end 109.734481 190.065519) (width 0.25) (layer "F.Cu") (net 7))
 (segment (start 109.734481 190.065519) (end 109.981969 190.065519) (width 0.25) (layer "B.Cu") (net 7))
 (segment (start 109.981969 190.065519) (end 114.11695 194.2005) (width 0.25) (layer "B.Cu") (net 7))
 (segment (start 114.11695 194.2005) (end 114.625 194.2005) (width 0.25) (layer "B.Cu") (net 7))
 (segment (start 114.625 194.2005) (end 114.8 194.3755) (width 0.25) (layer "B.Cu") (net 7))
 (segment (start 114.8 194.3755) (end 114.781969 194.265519) (width 0.25) (layer "F.Cu") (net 7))
 (segment (start 114.781969 194.265519) (end 115.674134 195.157684) (width 0.25) (layer "F.Cu") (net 7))
 (segment (start 116.6175 197.2) (end 116.6175 196.9995) (width 0.25) (layer "F.Cu") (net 7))
 (segment (start 116.6175 196.9995) (end 117.31695 196.9995) (width 0.25) (layer "F.Cu") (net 7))
 (segment (start 117.31695 196.9995) (end 118.9995 195.31695) (width 0.25) (layer "F.Cu") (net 7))
 (segment (start 118.9995 195.31695) (end 118.9995 193.11695) (width 0.25) (layer "F.Cu") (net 7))
 (segment (start 118.9995 193.11695) (end 119.503174 192.613276) (width 0.25) (layer "F.Cu") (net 7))
 (segment (start 119.503174 192.613276) (end 119.503174 192.513276) (width 0.25) (layer "F.Cu") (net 7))
 (segment (start 109.078245 189.141775) (end 108.97002 189.25) (width 0.25) (layer "F.Cu") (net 7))
 (segment (start 108.97002 189.25) (end 108.15 189.25) (width 0.25) (layer "F.Cu") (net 7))
 (segment (start 115.674134 195.157684) (end 114.89195 194.3755) (width 0.25) (layer "F.Cu") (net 7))
 (segment (start 114.89195 194.3755) (end 114.8 194.3755) (width 0.25) (layer "F.Cu") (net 7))
 (segment (start 120.755 191.135) (end 120.49 191.4) (width 0.25) (layer "F.Cu") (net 7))
 (segment (start 120.49 191.4) (end 120 191.4) (width 0.25) (layer "F.Cu") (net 7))
 (segment (start 120 191.4) (end 119.4 192) (width 0.25) (layer "F.Cu") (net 7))
 (segment (start 119.4 192) (end 119.4 192.2) (width 0.25) (layer "F.Cu") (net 7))
 (segment (start 119.503174 192.513276) (end 119.503174 192.113276) (width 0.25) (layer "F.Cu") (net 7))
 (segment (start 119.503174 192.113276) (end 119.4 192.2) (width 0.25) (layer "F.Cu") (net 7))
 (segment (start 116.4 197.2) (end 114.8 195.6) (width 0.25) (layer "B.Cu") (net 7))
 (segment (start 114.8 195.6) (end 114.8 194.4) (width 0.25) (layer "B.Cu") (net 7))
 (via (at 106 187.8) (size 0.6) (drill 0.3) (layers "F.Cu" "B.Cu") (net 6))
 (via (at 106.4 190) (size 0.6) (drill 0.3) (layers "F.Cu" "B.Cu") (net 6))
 (via (at 110.265519 189.534481) (size 0.6) (drill 0.3) (layers "F.Cu" "B.Cu") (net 6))
 (via (at 118.4 196.8) (size 0.6) (drill 0.3) (layers "F.Cu" "B.Cu") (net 6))
 (via (at 117 195.4) (size 0.6) (drill 0.3) (layers "F.Cu" "B.Cu") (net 6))
 (via (at 109.4 188.6) (size 0.6) (drill 0.3) (layers "F.Cu" "B.Cu") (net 6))
 (via (at 109.734481 190.065519) (size 0.6) (drill 0.3) (layers "F.Cu" "B.Cu") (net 7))
 (via (at 114.8 194.3755) (size 0.6) (drill 0.3) (layers "F.Cu" "B.Cu") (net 7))
 (via (at 116.4 197.2) (size 0.6) (drill 0.3) (layers "F.Cu" "B.Cu") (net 7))
 (segment (start 111.705 191.75) (end 110.755 192.7) (width 0.25) (layer "F.Cu") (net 2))
 (segment (start 110.755 192.7) (end 108.15 192.7) (width 0.25) (layer "F.Cu") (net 2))
 (segment (start 108.15 192.7) (end 107.575 193.275) (width 0.25) (layer "F.Cu") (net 2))
 (segment (start 107.575 193.275) (end 107.575 193.82) (width 0.25) (layer "F.Cu") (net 2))
 (segment (start 107.575 193.82) (end 107.2 194.195) (width 0.25) (layer "F.Cu") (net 2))
 (segment (start 107.2 194.195) (end 107.2 196.4) (width 0.25) (layer "F.Cu") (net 2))
 (segment (start 107.2 196.4) (end 107.22 196.42) (width 0.25) (layer "F.Cu") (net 2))
 (segment (start 107.22 196.42) (end 107.22 196.75) (width 0.25) (layer "F.Cu") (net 2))
 (segment (start 107.575 193.82) (end 107.8 193.595) (width 0.25) (layer "B.Cu") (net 2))
 (segment (start 107.8 193.595) (end 107.8 185.405) (width 0.25) (layer "B.Cu") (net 2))
 (segment (start 107.8 185.405) (end 107.575 185.18) (width 0.25) (layer "B.Cu") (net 2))
 (segment (start 107.575 185.18) (end 108.15 185.755) (width 0.25) (layer "F.Cu") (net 2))
 (segment (start 108.15 185.755) (end 108.15 186.3) (width 0.25) (layer "F.Cu") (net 2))
 (segment (start 107.575 185.18) (end 107.8 184.955) (width 0.25) (layer "F.Cu") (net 2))
 (segment (start 107.8 184.955) (end 107.8 183.2) (width 0.25) (layer "F.Cu") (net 2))
 (segment (start 107.8 183.2) (end 107.4 182.8) (width 0.25) (layer "F.Cu") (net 2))
 (segment (start 107.4 182.8) (end 107.2 182.8) (width 0.25) (layer "F.Cu") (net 2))
 (segment (start 107.2 182.8) (end 106.98 182.58) (width 0.25) (layer "F.Cu") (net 2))
 (segment (start 106.98 182.58) (end 106.98 182.49) (width 0.25) (layer "F.Cu") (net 2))
 (segment (start 106.98 182.49) (end 107.2 182.27) (width 0.25) (layer "F.Cu") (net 2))
 (segment (start 107.2 182.27) (end 107.2 182.2) (width 0.25) (layer "F.Cu") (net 2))
 (segment (start 107.2 182.2) (end 110.98 178.42) (width 0.25) (layer "F.Cu") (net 2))
 (segment (start 110.98 178.42) (end 110.98 177) (width 0.25) (layer "F.Cu") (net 2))
 (segment (start 116.6 176.2) (end 116.8 176) (width 0.25) (layer "F.Cu") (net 2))
 (segment (start 117.48 175.19) (end 120.0025 177.7125) (width 0.25) (layer "F.Cu") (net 2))
 (segment (start 120.0025 177.7125) (end 121.98 177.7125) (width 0.25) (layer "F.Cu") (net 2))
 (segment (start 111.705 191.75) (end 111.705 196.105) (width 0.25) (layer "F.Cu") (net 2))
 (segment (start 111.705 196.105) (end 113.6 198) (width 0.25) (layer "F.Cu") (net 2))
 (segment (start 113.6 198) (end 115 198) (width 0.25) (layer "F.Cu") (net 2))
 (segment (start 115 198) (end 115.6 197.4) (width 0.25) (layer "F.Cu") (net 2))
 (segment (start 115.6 197.4) (end 115.6 196.8) (width 0.25) (layer "F.Cu") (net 2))
 (segment (start 115.6 196.8) (end 116 196.4) (width 0.25) (layer "F.Cu") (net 2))
 (segment (start 116 196.4) (end 116.15 196.25) (width 0.25) (layer "F.Cu") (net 2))
 (segment (start 116.15 196.25) (end 116.6175 196.25) (width 0.25) (layer "F.Cu") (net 2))
 (segment (start 116.6175 196.25) (end 117.15 196.25) (width 0.25) (layer "F.Cu") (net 2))
 (segment (start 117.15 196.25) (end 117.8 195.6) (width 0.25) (layer "F.Cu") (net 2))
 (segment (start 117.8 195.6) (end 117.8 193.4) (width 0.25) (layer "F.Cu") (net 2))
 (segment (start 117.8 193.4) (end 117 192.6) (width 0.25) (layer "F.Cu") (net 2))
 (segment (start 117 192.6) (end 117 192) (width 0.25) (layer "F.Cu") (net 2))
 (segment (start 117 192) (end 116.4 191.4) (width 0.25) (layer "F.Cu") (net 2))
 (segment (start 116.4 191.4) (end 116.25 191.25) (width 0.25) (layer "F.Cu") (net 2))
 (segment (start 116.25 191.25) (end 115.8425 191.25) (width 0.25) (layer "F.Cu") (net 2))
 (segment (start 121.98 177.7125) (end 128.8 184.5325) (width 0.25) (layer "F.Cu") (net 2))
 (segment (start 128.8 184.5325) (end 128.8 186) (width 0.25) (layer "F.Cu") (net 2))
 (segment (start 128.8 186) (end 128.07 186.73) (width 0.25) (layer "F.Cu") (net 2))
 (segment (start 128.07 186.73) (end 127.98 186.73) (width 0.25) (layer "F.Cu") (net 2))
 (segment (start 116.2 176.2) (end 116.2 180.8) (width 0.25) (layer "F.Cu") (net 2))
 (segment (start 116.2 180.8) (end 117 181.6) (width 0.25) (layer "F.Cu") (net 2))
 (segment (start 117 181.6) (end 118 181.6) (width 0.25) (layer "F.Cu") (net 2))
 (segment (start 118 181.6) (end 120 183.6) (width 0.25) (layer "F.Cu") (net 2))
 (segment (start 120 183.6) (end 120 185.3) (width 0.25) (layer "F.Cu") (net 2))
 (segment (start 120 185.3) (end 120.755 186.055) (width 0.25) (layer "F.Cu") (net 2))
 (segment (start 120.755 186.055) (end 119.2 186.055) (width 0.25) (layer "F.Cu") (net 2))
 (segment (start 119.2 186.055) (end 118.255 187) (width 0.25) (layer "F.Cu") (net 2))
 (segment (start 113.705 192.2) (end 114.8 192.2) (width 0.25) (layer "F.Cu") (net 1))
 (segment (start 114.8 192.2) (end 115.8425 192.2) (width 0.25) (layer "F.Cu") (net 1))
 (segment (start 112.405 190.9) (end 111.3 190.9) (width 0.25) (layer "F.Cu") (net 1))
 (segment (start 111.3 190.9) (end 109.7 190.9) (width 0.25) (layer "F.Cu") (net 1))
 (segment (start 111.8 176.2) (end 116.2 176.2) (width 0.25) (layer "F.Cu") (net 2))
 (segment (start 116.2 176.2) (end 116.6 176.2) (width 0.25) (layer "F.Cu") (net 2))
 (segment (start 114.8 192) (end 114.8 192.2) (width 0.25) (layer "F.Cu") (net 1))
 (segment (start 108.24 196.75) (end 107.39 197.6) (width 0.25) (layer "F.Cu") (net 8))
 (segment (start 107.39 197.6) (end 107 197.6) (width 0.25) (layer "F.Cu") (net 8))
 (segment (start 107 197.6) (end 106 196.6) (width 0.25) (layer "F.Cu") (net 8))
 (segment (start 106 196.6) (end 106 192.4) (width 0.25) (layer "F.Cu") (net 8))
 (segment (start 106 192.4) (end 107.15 191.25) (width 0.25) (layer "F.Cu") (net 8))
 (segment (start 107.15 191.25) (end 108.15 191.25) (width 0.25) (layer "F.Cu") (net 8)))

